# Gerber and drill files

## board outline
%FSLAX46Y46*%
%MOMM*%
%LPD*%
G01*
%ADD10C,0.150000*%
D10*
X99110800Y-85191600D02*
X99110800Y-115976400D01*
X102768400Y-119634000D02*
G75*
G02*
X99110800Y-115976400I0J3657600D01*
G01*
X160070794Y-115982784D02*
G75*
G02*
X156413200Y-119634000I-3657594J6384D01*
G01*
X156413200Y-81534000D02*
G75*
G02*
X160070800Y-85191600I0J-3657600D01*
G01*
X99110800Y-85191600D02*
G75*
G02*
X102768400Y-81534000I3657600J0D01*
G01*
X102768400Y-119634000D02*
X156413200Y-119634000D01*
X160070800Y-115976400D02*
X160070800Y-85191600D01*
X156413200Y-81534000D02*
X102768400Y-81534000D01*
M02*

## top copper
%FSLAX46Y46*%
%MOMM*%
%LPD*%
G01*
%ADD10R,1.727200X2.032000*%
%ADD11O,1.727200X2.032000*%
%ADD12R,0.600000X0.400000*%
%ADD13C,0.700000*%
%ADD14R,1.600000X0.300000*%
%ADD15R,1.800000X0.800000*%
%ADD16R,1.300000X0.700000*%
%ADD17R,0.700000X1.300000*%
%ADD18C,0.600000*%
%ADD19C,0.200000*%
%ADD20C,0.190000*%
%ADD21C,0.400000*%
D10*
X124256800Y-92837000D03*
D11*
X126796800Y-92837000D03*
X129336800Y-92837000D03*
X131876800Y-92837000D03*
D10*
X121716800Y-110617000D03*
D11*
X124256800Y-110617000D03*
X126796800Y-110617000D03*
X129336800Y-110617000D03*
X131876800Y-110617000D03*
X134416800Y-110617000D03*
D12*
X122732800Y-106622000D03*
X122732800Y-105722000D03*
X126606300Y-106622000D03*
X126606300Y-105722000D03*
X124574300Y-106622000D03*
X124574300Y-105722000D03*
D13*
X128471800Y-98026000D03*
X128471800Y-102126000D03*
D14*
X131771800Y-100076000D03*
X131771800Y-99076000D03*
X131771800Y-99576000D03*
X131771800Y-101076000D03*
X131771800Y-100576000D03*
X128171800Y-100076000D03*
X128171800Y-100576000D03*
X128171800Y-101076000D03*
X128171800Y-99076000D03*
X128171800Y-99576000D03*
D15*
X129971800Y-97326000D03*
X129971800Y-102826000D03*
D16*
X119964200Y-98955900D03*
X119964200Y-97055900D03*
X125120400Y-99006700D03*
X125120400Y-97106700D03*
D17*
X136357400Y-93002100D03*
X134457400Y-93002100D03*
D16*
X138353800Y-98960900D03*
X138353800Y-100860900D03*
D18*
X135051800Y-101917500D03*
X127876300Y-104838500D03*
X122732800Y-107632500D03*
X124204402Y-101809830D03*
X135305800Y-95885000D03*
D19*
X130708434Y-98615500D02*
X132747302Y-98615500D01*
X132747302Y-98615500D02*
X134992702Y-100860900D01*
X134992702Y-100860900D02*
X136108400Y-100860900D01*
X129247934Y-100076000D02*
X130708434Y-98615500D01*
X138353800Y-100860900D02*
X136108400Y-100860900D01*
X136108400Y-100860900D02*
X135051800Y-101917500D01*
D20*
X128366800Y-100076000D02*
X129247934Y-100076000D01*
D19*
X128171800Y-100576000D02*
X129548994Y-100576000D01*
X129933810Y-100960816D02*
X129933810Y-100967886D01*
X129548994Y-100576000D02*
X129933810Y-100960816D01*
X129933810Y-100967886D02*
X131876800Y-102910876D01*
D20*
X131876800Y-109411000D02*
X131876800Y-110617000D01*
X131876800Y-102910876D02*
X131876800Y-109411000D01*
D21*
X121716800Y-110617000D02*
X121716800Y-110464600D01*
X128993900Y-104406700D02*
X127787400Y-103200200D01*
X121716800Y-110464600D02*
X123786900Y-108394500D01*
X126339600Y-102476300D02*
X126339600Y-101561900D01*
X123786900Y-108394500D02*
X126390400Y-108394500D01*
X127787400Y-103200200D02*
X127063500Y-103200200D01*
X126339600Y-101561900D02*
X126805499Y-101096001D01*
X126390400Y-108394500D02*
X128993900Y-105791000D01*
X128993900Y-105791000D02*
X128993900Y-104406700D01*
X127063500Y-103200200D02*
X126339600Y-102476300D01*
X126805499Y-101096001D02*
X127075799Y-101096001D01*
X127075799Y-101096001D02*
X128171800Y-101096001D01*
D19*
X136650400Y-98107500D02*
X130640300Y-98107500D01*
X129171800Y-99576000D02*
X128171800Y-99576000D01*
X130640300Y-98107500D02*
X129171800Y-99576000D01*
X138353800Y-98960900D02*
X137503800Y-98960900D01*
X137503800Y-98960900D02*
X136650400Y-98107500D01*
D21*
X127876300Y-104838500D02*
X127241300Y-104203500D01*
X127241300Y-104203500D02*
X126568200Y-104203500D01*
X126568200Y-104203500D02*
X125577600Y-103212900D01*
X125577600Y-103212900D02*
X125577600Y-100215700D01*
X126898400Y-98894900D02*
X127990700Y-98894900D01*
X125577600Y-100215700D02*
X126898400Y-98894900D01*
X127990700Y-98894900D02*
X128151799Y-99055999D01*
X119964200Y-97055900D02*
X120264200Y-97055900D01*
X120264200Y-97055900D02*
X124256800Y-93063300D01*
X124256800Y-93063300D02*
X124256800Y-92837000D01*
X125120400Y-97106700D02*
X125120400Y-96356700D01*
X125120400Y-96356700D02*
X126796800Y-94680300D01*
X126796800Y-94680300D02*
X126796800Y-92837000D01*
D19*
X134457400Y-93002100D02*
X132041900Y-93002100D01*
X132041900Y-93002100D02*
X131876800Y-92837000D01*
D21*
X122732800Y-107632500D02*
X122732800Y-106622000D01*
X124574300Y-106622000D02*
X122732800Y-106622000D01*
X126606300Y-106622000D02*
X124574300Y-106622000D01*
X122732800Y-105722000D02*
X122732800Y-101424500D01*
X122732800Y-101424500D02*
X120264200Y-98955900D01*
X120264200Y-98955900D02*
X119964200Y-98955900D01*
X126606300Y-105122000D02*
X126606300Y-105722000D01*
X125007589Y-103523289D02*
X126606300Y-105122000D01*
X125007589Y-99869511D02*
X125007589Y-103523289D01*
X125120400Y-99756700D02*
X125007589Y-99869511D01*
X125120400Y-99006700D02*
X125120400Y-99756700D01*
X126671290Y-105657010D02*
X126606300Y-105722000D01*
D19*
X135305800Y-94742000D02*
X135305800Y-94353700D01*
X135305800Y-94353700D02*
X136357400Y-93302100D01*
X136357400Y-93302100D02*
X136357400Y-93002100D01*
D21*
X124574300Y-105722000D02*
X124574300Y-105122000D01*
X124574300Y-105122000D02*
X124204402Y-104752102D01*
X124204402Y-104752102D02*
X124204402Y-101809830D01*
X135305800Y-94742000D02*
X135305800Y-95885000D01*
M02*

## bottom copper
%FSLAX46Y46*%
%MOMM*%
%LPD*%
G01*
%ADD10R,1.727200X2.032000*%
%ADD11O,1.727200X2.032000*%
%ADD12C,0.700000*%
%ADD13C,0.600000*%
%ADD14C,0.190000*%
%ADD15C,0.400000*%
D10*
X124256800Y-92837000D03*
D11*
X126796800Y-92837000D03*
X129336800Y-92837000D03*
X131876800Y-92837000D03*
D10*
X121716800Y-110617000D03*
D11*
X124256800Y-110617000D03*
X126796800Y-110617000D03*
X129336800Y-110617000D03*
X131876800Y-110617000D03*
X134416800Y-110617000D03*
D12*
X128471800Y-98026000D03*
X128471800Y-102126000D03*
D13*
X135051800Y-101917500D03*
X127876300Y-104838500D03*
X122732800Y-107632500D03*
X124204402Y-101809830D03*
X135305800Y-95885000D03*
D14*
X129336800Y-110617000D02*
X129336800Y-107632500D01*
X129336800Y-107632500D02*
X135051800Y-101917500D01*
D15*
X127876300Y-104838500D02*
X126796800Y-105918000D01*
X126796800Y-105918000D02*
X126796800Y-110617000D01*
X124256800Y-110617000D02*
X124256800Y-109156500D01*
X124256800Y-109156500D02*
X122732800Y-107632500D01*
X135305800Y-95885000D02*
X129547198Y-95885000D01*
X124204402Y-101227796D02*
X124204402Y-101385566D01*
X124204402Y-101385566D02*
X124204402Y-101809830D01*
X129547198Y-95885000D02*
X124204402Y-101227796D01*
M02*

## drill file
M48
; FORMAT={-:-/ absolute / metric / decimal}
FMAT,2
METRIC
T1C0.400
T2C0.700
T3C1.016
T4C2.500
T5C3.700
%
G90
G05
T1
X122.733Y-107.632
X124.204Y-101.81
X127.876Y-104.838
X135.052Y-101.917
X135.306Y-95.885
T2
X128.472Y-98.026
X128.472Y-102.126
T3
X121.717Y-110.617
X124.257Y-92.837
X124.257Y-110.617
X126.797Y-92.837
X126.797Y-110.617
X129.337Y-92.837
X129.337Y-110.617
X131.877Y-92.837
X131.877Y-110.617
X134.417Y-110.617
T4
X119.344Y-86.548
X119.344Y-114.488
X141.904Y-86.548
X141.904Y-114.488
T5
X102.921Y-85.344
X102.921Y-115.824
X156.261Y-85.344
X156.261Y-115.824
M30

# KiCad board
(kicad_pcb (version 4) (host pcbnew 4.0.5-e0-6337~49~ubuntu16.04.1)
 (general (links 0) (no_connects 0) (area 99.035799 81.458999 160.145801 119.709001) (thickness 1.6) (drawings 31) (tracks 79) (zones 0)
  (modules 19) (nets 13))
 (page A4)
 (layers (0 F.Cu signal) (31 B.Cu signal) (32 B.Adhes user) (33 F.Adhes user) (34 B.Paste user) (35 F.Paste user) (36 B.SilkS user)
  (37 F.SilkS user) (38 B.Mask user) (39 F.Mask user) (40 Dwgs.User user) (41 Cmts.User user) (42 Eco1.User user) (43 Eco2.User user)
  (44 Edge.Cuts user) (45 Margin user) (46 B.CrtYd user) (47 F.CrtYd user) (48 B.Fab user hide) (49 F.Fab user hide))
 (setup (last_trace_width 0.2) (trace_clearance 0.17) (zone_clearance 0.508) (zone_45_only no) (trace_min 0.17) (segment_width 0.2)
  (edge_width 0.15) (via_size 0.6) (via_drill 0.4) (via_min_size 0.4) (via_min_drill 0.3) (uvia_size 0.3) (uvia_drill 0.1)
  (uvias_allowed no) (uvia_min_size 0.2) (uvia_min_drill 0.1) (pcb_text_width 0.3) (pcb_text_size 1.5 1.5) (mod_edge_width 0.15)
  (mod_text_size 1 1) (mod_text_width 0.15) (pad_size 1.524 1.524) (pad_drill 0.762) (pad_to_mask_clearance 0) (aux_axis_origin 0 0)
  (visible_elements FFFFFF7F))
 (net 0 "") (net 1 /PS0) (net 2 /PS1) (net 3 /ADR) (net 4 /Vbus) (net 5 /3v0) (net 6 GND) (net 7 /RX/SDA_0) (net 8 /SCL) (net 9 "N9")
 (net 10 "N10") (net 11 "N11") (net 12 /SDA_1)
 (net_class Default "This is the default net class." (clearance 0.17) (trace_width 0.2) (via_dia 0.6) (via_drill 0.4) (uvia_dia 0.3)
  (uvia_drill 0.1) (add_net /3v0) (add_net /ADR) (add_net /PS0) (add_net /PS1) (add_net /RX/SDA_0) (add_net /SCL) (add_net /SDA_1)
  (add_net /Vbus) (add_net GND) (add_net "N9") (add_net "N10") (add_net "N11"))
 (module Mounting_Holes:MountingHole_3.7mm (layer F.Cu) (at 156.2608 115.824)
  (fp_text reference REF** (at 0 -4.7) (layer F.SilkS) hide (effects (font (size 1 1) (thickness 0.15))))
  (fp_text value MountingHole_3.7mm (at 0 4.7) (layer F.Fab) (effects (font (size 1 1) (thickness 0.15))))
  (pad 1 np_thru_hole circle (at 0 0) (size 3.7 3.7) (drill 3.7) (layers *.Cu *.Mask)))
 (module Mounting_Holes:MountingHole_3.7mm (layer F.Cu) (at 156.2608 85.344)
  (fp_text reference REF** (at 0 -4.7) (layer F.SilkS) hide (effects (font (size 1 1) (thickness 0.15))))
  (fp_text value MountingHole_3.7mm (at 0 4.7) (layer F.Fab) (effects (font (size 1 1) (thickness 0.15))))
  (pad 1 np_thru_hole circle (at 0 0) (size 3.7 3.7) (drill 3.7) (layers *.Cu *.Mask)))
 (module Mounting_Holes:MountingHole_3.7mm (layer F.Cu) (at 102.9208 115.824)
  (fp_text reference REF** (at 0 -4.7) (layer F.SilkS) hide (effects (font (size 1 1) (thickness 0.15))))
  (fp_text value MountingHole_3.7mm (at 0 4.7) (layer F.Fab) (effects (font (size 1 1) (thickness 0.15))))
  (pad 1 np_thru_hole circle (at 0 0) (size 3.7 3.7) (drill 3.7) (layers *.Cu *.Mask)))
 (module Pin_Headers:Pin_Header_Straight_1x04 (layer F.Cu) (at 124.2568 92.837 90)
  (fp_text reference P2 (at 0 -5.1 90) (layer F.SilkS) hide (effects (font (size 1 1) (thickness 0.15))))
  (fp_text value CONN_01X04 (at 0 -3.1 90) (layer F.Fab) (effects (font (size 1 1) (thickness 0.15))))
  (pad 1 thru_hole rect (at 0 0 90) (size 2.032 1.7272) (drill 1.016) (layers *.Cu *.Mask) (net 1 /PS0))
  (pad 2 thru_hole oval (at 0 2.54 90) (size 2.032 1.7272) (drill 1.016) (layers *.Cu *.Mask) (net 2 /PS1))
  (pad 3 thru_hole oval (at 0 5.08 90) (size 2.032 1.7272) (drill 1.016) (layers *.Cu *.Mask))
  (pad 4 thru_hole oval (at 0 7.62 90) (size 2.032 1.7272) (drill 1.016) (layers *.Cu *.Mask) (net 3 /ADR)))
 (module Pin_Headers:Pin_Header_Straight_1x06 (layer F.Cu) (at 121.7168 110.617 90)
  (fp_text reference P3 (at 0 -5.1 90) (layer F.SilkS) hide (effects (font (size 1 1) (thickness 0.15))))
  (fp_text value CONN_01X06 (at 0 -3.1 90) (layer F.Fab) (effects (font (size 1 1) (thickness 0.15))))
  (pad 1 thru_hole rect (at 0 0 90) (size 2.032 1.7272) (drill 1.016) (layers *.Cu *.Mask) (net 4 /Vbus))
  (pad 2 thru_hole oval (at 0 2.54 90) (size 2.032 1.7272) (drill 1.016) (layers *.Cu *.Mask) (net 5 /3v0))
  (pad 3 thru_hole oval (at 0 5.08 90) (size 2.032 1.7272) (drill 1.016) (layers *.Cu *.Mask) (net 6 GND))
  (pad 4 thru_hole oval (at 0 7.62 90) (size 2.032 1.7272) (drill 1.016) (layers *.Cu *.Mask) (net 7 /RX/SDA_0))
  (pad 5 thru_hole oval (at 0 10.16 90) (size 2.032 1.7272) (drill 1.016) (layers *.Cu *.Mask) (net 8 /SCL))
  (pad 6 thru_hole oval (at 0 12.7 90) (size 2.032 1.7272) (drill 1.016) (layers *.Cu *.Mask)))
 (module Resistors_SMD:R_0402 (layer F.Cu) (at 122.7328 106.172 90)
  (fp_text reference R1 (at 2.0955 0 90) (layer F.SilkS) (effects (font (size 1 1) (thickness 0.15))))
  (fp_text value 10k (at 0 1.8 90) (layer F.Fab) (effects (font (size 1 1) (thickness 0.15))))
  (pad 1 smd rect (at -0.45 0 90) (size 0.4 0.6) (layers F.Cu F.Paste F.Mask) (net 5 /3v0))
  (pad 2 smd rect (at 0.45 0 90) (size 0.4 0.6) (layers F.Cu F.Paste F.Mask) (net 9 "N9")))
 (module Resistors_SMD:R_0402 (layer F.Cu) (at 126.6063 106.172 90)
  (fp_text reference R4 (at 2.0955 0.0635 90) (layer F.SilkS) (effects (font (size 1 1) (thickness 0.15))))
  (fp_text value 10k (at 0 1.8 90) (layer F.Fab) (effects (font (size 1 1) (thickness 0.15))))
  (pad 1 smd rect (at -0.45 0 90) (size 0.4 0.6) (layers F.Cu F.Paste F.Mask) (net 5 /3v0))
  (pad 2 smd rect (at 0.45 0 90) (size 0.4 0.6) (layers F.Cu F.Paste F.Mask) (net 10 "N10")))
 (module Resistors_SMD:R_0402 (layer F.Cu) (at 124.5743 106.172 90)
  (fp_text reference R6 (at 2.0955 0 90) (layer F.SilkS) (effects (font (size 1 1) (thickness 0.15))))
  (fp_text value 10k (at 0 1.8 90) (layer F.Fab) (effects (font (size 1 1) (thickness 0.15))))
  (pad 1 smd rect (at -0.45 0 90) (size 0.4 0.6) (layers F.Cu F.Paste F.Mask) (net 5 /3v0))
  (pad 2 smd rect (at 0.45 0 90) (size 0.4 0.6) (layers F.Cu F.Paste F.Mask) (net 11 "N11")))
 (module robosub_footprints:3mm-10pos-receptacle (layer F.Cu) (at 129.9718 100.076 90)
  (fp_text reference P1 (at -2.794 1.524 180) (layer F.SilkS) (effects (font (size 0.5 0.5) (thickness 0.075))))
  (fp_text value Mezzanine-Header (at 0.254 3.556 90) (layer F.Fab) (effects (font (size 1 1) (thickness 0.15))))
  (pad "" thru_hole circle (at 2.05 -1.5 90) (size 0.7 0.7) (drill 0.7) (layers *.Cu *.Mask))
  (pad "" thru_hole circle (at -2.05 -1.5 90) (size 0.7 0.7) (drill 0.7) (layers *.Cu *.Mask))
  (pad 6 smd rect (at 0 1.8 90) (size 0.3 1.6) (layers F.Cu F.Paste F.Mask))
  (pad 10 smd rect (at 1 1.8 90) (size 0.3 1.6) (layers F.Cu F.Paste F.Mask))
  (pad 8 smd rect (at 0.5 1.8 90) (size 0.3 1.6) (layers F.Cu F.Paste F.Mask))
  (pad 2 smd rect (at -1 1.8 90) (size 0.3 1.6) (layers F.Cu F.Paste F.Mask))
  (pad 4 smd rect (at -0.5 1.8 90) (size 0.3 1.6) (layers F.Cu F.Paste F.Mask))
  (pad 5 smd rect (at 0 -1.8 90) (size 0.3 1.6) (layers F.Cu F.Paste F.Mask) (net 7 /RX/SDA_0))
  (pad 3 smd rect (at -0.5 -1.8 90) (size 0.3 1.6) (layers F.Cu F.Paste F.Mask) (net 8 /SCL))
  (pad 1 smd rect (at -1 -1.8 90) (size 0.3 1.6) (layers F.Cu F.Paste F.Mask) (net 4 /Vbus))
  (pad 9 smd rect (at 1 -1.8 90) (size 0.3 1.6) (layers F.Cu F.Paste F.Mask) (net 6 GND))
  (pad 7 smd rect (at 0.5 -1.8 90) (size 0.3 1.6) (layers F.Cu F.Paste F.Mask) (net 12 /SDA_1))
  (pad "" smd rect (at 2.75 0 90) (size 0.8 1.8) (layers F.Cu F.Paste F.Mask))
  (pad "" smd rect (at -2.75 0 90) (size 0.8 1.8) (layers F.Cu F.Paste F.Mask)))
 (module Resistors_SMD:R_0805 (layer F.Cu) (at 119.9642 98.0059 90)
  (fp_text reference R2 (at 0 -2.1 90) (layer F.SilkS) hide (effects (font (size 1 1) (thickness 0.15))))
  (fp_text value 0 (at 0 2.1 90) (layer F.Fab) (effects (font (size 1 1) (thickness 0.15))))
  (pad 1 smd rect (at -0.95 0 90) (size 0.7 1.3) (layers F.Cu F.Paste F.Mask) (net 9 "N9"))
  (pad 2 smd rect (at 0.95 0 90) (size 0.7 1.3) (layers F.Cu F.Paste F.Mask) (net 1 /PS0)))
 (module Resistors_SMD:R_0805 (layer F.Cu) (at 125.1204 98.0567 90)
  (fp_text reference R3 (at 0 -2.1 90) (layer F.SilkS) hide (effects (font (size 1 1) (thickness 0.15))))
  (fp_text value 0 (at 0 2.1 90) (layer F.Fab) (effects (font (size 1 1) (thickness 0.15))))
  (pad 1 smd rect (at -0.95 0 90) (size 0.7 1.3) (layers F.Cu F.Paste F.Mask) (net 10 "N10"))
  (pad 2 smd rect (at 0.95 0 90) (size 0.7 1.3) (layers F.Cu F.Paste F.Mask) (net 2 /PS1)))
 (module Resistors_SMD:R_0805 (layer F.Cu) (at 135.4074 93.0021 180)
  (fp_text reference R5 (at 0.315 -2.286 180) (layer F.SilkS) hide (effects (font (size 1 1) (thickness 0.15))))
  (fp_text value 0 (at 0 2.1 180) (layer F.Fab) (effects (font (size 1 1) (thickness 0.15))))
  (pad 1 smd rect (at -0.95 0 180) (size 0.7 1.3) (layers F.Cu F.Paste F.Mask) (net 11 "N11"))
  (pad 2 smd rect (at 0.95 0 180) (size 0.7 1.3) (layers F.Cu F.Paste F.Mask) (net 3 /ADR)))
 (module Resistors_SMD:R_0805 (layer F.Cu) (at 138.3538 99.9109 270)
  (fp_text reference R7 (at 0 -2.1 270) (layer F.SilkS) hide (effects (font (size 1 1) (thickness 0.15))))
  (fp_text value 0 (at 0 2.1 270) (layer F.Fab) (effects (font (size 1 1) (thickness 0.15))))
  (pad 1 smd rect (at -0.95 0 270) (size 0.7 1.3) (layers F.Cu F.Paste F.Mask) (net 12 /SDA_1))
  (pad 2 smd rect (at 0.95 0 270) (size 0.7 1.3) (layers F.Cu F.Paste F.Mask) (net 7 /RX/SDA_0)))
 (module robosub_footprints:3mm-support (layer F.Cu) (at 141.9042 86.548204)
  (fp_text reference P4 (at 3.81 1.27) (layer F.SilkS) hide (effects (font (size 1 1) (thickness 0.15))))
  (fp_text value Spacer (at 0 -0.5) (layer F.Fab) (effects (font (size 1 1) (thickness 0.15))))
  (pad "" np_thru_hole circle (at 0 0) (size 2.5 2.5) (drill 2.5) (layers *.Cu *.Mask)))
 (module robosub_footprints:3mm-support (layer F.Cu) (at 119.3442 114.488204)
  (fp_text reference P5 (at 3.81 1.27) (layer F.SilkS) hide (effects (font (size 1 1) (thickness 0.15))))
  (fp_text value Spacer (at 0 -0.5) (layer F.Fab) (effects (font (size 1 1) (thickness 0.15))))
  (pad "" np_thru_hole circle (at 0 0) (size 2.5 2.5) (drill 2.5) (layers *.Cu *.Mask)))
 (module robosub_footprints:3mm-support (layer F.Cu) (at 119.3442 86.548204)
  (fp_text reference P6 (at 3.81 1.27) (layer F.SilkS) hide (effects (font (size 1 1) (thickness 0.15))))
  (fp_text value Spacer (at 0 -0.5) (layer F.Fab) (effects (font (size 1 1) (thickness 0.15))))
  (pad "" np_thru_hole circle (at 0 0) (size 2.5 2.5) (drill 2.5) (layers *.Cu *.Mask)))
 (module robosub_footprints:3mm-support (layer F.Cu) (at 141.9042 114.488204)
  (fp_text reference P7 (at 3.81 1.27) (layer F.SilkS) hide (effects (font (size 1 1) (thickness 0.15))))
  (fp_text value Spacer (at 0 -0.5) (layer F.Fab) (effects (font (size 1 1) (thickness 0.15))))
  (pad "" np_thru_hole circle (at 0 0) (size 2.5 2.5) (drill 2.5) (layers *.Cu *.Mask)))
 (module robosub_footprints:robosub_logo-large (layer F.Cu) (at 155.3718 101.3714 90)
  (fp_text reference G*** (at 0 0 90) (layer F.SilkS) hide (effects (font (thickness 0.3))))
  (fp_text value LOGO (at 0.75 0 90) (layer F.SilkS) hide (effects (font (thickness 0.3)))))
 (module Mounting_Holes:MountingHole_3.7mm (layer F.Cu) (at 102.9208 85.344)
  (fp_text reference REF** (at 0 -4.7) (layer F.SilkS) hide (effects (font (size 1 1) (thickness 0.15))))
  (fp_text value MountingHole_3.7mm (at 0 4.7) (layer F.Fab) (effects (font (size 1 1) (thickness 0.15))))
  (pad 1 np_thru_hole circle (at 0 0) (size 3.7 3.7) (drill 3.7) (layers *.Cu *.Mask)))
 (gr_line (start 99.1108 85.1916) (end 99.1108 115.9764) (layer Edge.Cuts) (width 0.15))
 (gr_arc (start 102.7684 115.9764) (end 99.1108 115.9764) (angle -90) (layer Edge.Cuts) (width 0.15))
 (gr_arc (start 156.4132 115.9764) (end 156.4132 119.634) (angle -89.9) (layer Edge.Cuts) (width 0.15))
 (gr_arc (start 156.4132 85.1916) (end 160.0708 85.1916) (angle -90) (layer Edge.Cuts) (width 0.15))
 (gr_arc (start 102.7684 85.1916) (end 102.7684 81.534) (angle -90) (layer Edge.Cuts) (width 0.15))
 (gr_line (start 102.7684 119.634) (end 156.4132 119.634) (layer Edge.Cuts) (width 0.15))
 (gr_line (start 160.0708 115.9764) (end 160.0708 85.1916) (layer Edge.Cuts) (width 0.15))
 (gr_line (start 156.4132 81.534) (end 102.7684 81.534) (layer Edge.Cuts) (width 0.15))
 (segment (start 130.708434 98.6155) (end 132.747302 98.6155) (width 0.2) (layer F.Cu) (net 7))
 (segment (start 132.747302 98.6155) (end 134.992702 100.8609) (width 0.2) (layer F.Cu) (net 7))
 (segment (start 134.992702 100.8609) (end 136.1084 100.8609) (width 0.2) (layer F.Cu) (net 7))
 (segment (start 129.247934 100.076) (end 130.708434 98.6155) (width 0.2) (layer F.Cu) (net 7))
 (segment (start 138.3538 100.8609) (end 136.1084 100.8609) (width 0.2) (layer F.Cu) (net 7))
 (segment (start 136.1084 100.8609) (end 135.0518 101.9175) (width 0.2) (layer F.Cu) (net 7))
 (segment (start 129.3368 110.617) (end 129.3368 107.6325) (width 0.19) (layer B.Cu) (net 7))
 (segment (start 129.3368 107.6325) (end 135.0518 101.9175) (width 0.19) (layer B.Cu) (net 7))
 (via (at 135.0518 101.9175) (size 0.6) (drill 0.4) (layers F.Cu B.Cu) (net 7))
 (segment (start 128.3668 100.076) (end 129.247934 100.076) (width 0.19) (layer F.Cu) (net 7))
 (segment (start 128.1718 100.576) (end 129.548994 100.576) (width 0.2) (layer F.Cu) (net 8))
 (segment (start 129.93381 100.960816) (end 129.93381 100.967886) (width 0.2) (layer F.Cu) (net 8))
 (segment (start 129.548994 100.576) (end 129.93381 100.960816) (width 0.2) (layer F.Cu) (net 8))
 (segment (start 129.93381 100.967886) (end 131.8768 102.910876) (width 0.2) (layer F.Cu) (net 8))
 (segment (start 131.8768 109.411) (end 131.8768 110.617) (width 0.19) (layer F.Cu) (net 8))
 (segment (start 131.8768 102.910876) (end 131.8768 109.411) (width 0.19) (layer F.Cu) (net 8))
 (segment (start 121.7168 110.617) (end 121.7168 110.4646) (width 0.4) (layer F.Cu) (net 4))
 (segment (start 128.9939 104.4067) (end 127.7874 103.2002) (width 0.4) (layer F.Cu) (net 4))
 (segment (start 121.7168 110.4646) (end 123.7869 108.3945) (width 0.4) (layer F.Cu) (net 4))
 (segment (start 126.3396 102.4763) (end 126.3396 101.5619) (width 0.4) (layer F.Cu) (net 4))
 (segment (start 123.7869 108.3945) (end 126.3904 108.3945) (width 0.4) (layer F.Cu) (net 4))
 (segment (start 127.7874 103.2002) (end 127.0635 103.2002) (width 0.4) (layer F.Cu) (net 4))
 (segment (start 126.3396 101.5619) (end 126.805499 101.096001) (width 0.4) (layer F.Cu) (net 4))
 (segment (start 126.3904 108.3945) (end 128.9939 105.791) (width 0.4) (layer F.Cu) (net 4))
 (segment (start 128.9939 105.791) (end 128.9939 104.4067) (width 0.4) (layer F.Cu) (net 4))
 (segment (start 127.0635 103.2002) (end 126.3396 102.4763) (width 0.4) (layer F.Cu) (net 4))
 (segment (start 126.805499 101.096001) (end 127.075799 101.096001) (width 0.4) (layer F.Cu) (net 4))
 (segment (start 127.075799 101.096001) (end 128.1718 101.096001) (width 0.4) (layer F.Cu) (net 4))
 (segment (start 136.6504 98.1075) (end 130.6403 98.1075) (width 0.2) (layer F.Cu) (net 12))
 (segment (start 129.1718 99.576) (end 128.1718 99.576) (width 0.2) (layer F.Cu) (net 12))
 (segment (start 130.6403 98.1075) (end 129.1718 99.576) (width 0.2) (layer F.Cu) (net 12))
 (segment (start 138.3538 98.9609) (end 137.5038 98.9609) (width 0.2) (layer F.Cu) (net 12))
 (segment (start 137.5038 98.9609) (end 136.6504 98.1075) (width 0.2) (layer F.Cu) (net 12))
 (segment (start 127.8763 104.8385) (end 127.2413 104.2035) (width 0.4) (layer F.Cu) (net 6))
 (segment (start 127.2413 104.2035) (end 126.5682 104.2035) (width 0.4) (layer F.Cu) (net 6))
 (segment (start 126.5682 104.2035) (end 125.5776 103.2129) (width 0.4) (layer F.Cu) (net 6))
 (segment (start 125.5776 103.2129) (end 125.5776 100.2157) (width 0.4) (layer F.Cu) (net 6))
 (segment (start 126.8984 98.8949) (end 127.9907 98.8949) (width 0.4) (layer F.Cu) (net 6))
 (segment (start 125.5776 100.2157) (end 126.8984 98.8949) (width 0.4) (layer F.Cu) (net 6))
 (segment (start 127.9907 98.8949) (end 128.151799 99.055999) (width 0.4) (layer F.Cu) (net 6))
 (segment (start 127.8763 104.8385) (end 126.7968 105.918) (width 0.4) (layer B.Cu) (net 6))
 (segment (start 126.7968 105.918) (end 126.7968 110.617) (width 0.4) (layer B.Cu) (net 6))
 (via (at 127.8763 104.8385) (size 0.6) (drill 0.4) (layers F.Cu B.Cu) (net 6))
 (segment (start 119.9642 97.0559) (end 120.2642 97.0559) (width 0.4) (layer F.Cu) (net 1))
 (segment (start 120.2642 97.0559) (end 124.2568 93.0633) (width 0.4) (layer F.Cu) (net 1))
 (segment (start 124.2568 93.0633) (end 124.2568 92.837) (width 0.4) (layer F.Cu) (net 1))
 (segment (start 125.1204 97.1067) (end 125.1204 96.3567) (width 0.4) (layer F.Cu) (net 2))
 (segment (start 125.1204 96.3567) (end 126.7968 94.6803) (width 0.4) (layer F.Cu) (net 2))
 (segment (start 126.7968 94.6803) (end 126.7968 92.837) (width 0.4) (layer F.Cu) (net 2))
 (segment (start 134.4574 93.0021) (end 132.0419 93.0021) (width 0.2) (layer F.Cu) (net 3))
 (segment (start 132.0419 93.0021) (end 131.8768 92.837) (width 0.2) (layer F.Cu) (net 3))
 (segment (start 122.7328 107.6325) (end 122.7328 106.622) (width 0.4) (layer F.Cu) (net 5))
 (segment (start 124.2568 110.617) (end 124.2568 109.1565) (width 0.4) (layer B.Cu) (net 5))
 (segment (start 124.2568 109.1565) (end 122.7328 107.6325) (width 0.4) (layer B.Cu) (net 5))
 (via (at 122.7328 107.6325) (size 0.6) (drill 0.4) (layers F.Cu B.Cu) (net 5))
 (segment (start 124.5743 106.622) (end 122.7328 106.622) (width 0.4) (layer F.Cu) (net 5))
 (segment (start 126.6063 106.622) (end 124.5743 106.622) (width 0.4) (layer F.Cu) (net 5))
 (segment (start 122.7328 105.722) (end 122.7328 101.4245) (width 0.4) (layer F.Cu) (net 9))
 (segment (start 122.7328 101.4245) (end 120.2642 98.9559) (width 0.4) (layer F.Cu) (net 9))
 (segment (start 120.2642 98.9559) (end 119.9642 98.9559) (width 0.4) (layer F.Cu) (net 9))
 (segment (start 126.6063 105.122) (end 126.6063 105.722) (width 0.4) (layer F.Cu) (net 10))
 (segment (start 125.007589 103.523289) (end 126.6063 105.122) (width 0.4) (layer F.Cu) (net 10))
 (segment (start 125.007589 99.869511) (end 125.007589 103.523289) (width 0.4) (layer F.Cu) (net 10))
 (segment (start 125.1204 99.7567) (end 125.007589 99.869511) (width 0.4) (layer F.Cu) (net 10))
 (segment (start 125.1204 99.0067) (end 125.1204 99.7567) (width 0.4) (layer F.Cu) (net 10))
 (segment (start 126.67129 105.65701) (end 126.6063 105.722) (width 0.4) (layer F.Cu) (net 10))
 (segment (start 135.3058 94.742) (end 135.3058 94.3537) (width 0.2) (layer F.Cu) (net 11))
 (segment (start 135.3058 94.3537) (end 136.3574 93.3021) (width 0.2) (layer F.Cu) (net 11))
 (segment (start 136.3574 93.3021) (end 136.3574 93.0021) (width 0.2) (layer F.Cu) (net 11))
 (segment (start 135.3058 95.885) (end 129.547198 95.885) (width 0.4) (layer B.Cu) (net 11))
 (segment (start 124.204402 101.227796) (end 124.204402 101.385566) (width 0.4) (layer B.Cu) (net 11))
 (via (at 124.204402 101.80983) (size 0.6) (drill 0.4) (layers F.Cu B.Cu) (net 11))
 (segment (start 124.204402 101.385566) (end 124.204402 101.80983) (width 0.4) (layer B.Cu) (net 11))
 (segment (start 129.547198 95.885) (end 124.204402 101.227796) (width 0.4) (layer B.Cu) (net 11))
 (segment (start 124.5743 105.722) (end 124.5743 105.122) (width 0.4) (layer F.Cu) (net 11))
 (segment (start 124.5743 105.122) (end 124.204402 104.752102) (width 0.4) (layer F.Cu) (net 11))
 (segment (start 124.204402 104.752102) (end 124.204402 101.80983) (width 0.4) (layer F.Cu) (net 11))
 (segment (start 135.3058 94.742) (end 135.3058 95.885) (width 0.4) (layer F.Cu) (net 11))
 (via (at 135.3058 95.885) (size 0.6) (drill 0.4) (layers F.Cu B.Cu) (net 11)))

